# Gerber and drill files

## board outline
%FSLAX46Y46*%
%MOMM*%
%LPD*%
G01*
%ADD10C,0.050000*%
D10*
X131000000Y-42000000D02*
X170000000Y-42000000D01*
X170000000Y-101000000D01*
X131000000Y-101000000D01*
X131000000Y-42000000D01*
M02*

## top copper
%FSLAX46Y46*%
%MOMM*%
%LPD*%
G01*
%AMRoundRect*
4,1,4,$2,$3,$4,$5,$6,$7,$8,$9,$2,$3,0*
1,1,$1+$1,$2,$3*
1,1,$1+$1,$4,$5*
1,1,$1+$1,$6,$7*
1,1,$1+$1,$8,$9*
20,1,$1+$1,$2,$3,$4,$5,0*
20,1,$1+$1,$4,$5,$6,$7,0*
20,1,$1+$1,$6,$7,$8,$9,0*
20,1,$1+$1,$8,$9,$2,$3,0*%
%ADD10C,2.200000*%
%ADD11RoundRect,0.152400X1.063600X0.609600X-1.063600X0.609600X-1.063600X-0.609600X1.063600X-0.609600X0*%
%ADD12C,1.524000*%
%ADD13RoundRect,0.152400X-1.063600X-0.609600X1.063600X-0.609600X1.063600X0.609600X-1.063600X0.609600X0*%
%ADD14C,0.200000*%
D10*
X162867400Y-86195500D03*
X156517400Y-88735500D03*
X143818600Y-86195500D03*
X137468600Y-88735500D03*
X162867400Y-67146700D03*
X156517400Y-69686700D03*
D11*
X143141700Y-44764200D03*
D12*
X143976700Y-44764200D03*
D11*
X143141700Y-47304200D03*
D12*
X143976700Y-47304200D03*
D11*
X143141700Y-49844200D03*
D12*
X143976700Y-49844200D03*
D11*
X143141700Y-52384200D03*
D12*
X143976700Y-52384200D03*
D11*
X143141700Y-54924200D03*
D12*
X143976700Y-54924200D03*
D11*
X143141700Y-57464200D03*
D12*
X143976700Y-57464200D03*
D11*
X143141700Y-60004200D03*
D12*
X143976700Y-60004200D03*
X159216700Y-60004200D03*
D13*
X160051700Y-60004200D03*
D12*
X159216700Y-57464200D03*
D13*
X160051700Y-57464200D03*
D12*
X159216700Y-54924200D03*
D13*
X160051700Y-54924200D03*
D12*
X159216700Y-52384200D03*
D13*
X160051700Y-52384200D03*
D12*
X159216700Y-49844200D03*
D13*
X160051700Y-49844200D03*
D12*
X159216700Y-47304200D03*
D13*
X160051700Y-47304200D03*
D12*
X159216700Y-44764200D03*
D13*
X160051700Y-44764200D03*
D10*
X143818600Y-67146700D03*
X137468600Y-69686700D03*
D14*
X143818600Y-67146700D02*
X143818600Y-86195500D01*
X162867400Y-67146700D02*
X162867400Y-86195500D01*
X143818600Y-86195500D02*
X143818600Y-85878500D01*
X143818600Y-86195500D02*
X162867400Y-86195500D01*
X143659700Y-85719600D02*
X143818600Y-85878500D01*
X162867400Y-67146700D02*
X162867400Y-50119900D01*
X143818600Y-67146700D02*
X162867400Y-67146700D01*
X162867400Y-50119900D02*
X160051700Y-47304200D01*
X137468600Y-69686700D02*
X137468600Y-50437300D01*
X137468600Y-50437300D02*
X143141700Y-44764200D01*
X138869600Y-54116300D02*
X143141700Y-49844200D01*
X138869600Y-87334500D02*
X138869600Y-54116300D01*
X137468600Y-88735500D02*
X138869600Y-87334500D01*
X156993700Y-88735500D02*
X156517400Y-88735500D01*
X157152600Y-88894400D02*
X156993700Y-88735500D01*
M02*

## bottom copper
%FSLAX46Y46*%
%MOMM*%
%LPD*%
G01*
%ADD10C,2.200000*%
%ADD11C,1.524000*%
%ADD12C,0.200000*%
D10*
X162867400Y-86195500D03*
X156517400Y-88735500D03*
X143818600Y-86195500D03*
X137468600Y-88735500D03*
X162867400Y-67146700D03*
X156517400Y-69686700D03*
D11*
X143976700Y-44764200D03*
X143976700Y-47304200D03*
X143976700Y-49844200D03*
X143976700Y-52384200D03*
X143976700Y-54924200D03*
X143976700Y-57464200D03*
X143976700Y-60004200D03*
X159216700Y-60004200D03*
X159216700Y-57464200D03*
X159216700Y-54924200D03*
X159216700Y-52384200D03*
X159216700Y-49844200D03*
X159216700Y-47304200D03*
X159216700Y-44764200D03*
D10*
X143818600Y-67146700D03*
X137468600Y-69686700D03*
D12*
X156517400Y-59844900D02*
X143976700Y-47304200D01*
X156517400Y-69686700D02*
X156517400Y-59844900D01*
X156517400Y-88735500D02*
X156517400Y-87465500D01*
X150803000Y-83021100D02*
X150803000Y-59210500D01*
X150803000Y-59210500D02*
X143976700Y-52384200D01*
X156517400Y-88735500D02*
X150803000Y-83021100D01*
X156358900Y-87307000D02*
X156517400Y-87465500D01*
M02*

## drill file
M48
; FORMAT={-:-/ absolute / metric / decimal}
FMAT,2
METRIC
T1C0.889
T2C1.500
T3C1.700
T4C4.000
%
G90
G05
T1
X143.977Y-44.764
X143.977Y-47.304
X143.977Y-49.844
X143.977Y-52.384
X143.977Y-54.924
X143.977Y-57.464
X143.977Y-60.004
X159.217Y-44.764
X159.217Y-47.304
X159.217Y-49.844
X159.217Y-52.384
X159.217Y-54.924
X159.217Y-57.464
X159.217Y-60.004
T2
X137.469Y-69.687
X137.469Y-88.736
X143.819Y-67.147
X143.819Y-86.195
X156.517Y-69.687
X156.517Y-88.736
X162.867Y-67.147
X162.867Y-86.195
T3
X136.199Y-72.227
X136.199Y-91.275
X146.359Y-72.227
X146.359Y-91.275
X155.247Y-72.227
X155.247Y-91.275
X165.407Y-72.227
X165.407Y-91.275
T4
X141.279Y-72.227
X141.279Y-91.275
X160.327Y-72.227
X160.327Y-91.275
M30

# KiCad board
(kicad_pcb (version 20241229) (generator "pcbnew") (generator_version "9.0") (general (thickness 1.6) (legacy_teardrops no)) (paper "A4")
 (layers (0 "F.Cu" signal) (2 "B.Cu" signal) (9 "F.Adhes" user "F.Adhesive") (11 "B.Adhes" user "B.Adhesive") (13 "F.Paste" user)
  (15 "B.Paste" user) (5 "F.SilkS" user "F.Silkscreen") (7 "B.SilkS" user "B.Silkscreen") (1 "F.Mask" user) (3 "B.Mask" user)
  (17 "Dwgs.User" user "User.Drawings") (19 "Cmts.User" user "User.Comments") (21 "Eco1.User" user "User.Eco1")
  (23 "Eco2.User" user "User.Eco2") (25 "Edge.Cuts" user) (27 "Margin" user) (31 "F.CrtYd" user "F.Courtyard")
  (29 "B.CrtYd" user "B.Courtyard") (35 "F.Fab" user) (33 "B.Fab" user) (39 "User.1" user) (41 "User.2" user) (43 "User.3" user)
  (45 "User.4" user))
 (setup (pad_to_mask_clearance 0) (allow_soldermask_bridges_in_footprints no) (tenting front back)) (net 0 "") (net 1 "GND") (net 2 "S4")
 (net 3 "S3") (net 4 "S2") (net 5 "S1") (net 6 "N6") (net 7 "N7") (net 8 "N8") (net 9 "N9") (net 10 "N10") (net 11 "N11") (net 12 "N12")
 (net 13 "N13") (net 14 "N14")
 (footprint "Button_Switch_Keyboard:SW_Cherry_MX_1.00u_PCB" (layer "F.Cu") (at 162.8674 86.1955)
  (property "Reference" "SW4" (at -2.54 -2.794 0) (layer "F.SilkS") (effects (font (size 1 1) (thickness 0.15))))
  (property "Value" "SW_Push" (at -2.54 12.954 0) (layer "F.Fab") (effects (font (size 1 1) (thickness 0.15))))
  (pad "" np_thru_hole circle (at -7.62 5.08) (size 1.7 1.7) (drill 1.7) (layers "*.Cu" "*.Mask"))
  (pad "" np_thru_hole circle (at -2.54 5.08) (size 4 4) (drill 4) (layers "*.Cu" "*.Mask"))
  (pad "" np_thru_hole circle (at 2.54 5.08) (size 1.7 1.7) (drill 1.7) (layers "*.Cu" "*.Mask"))
  (pad "1" thru_hole circle (at 0 0) (size 2.2 2.2) (drill 1.5) (layers "*.Cu" "*.Mask") (remove_unused_layers no) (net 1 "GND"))
  (pad "2" thru_hole circle (at -6.35 2.54) (size 2.2 2.2) (drill 1.5) (layers "*.Cu" "*.Mask") (remove_unused_layers no) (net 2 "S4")))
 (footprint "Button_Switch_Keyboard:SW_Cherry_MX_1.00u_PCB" (layer "F.Cu") (at 143.8186 86.1955)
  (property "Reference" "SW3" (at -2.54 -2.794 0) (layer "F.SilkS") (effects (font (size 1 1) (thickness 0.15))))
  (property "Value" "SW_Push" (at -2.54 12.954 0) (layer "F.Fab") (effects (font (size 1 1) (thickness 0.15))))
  (pad "" np_thru_hole circle (at -7.62 5.08) (size 1.7 1.7) (drill 1.7) (layers "*.Cu" "*.Mask"))
  (pad "" np_thru_hole circle (at -2.54 5.08) (size 4 4) (drill 4) (layers "*.Cu" "*.Mask"))
  (pad "" np_thru_hole circle (at 2.54 5.08) (size 1.7 1.7) (drill 1.7) (layers "*.Cu" "*.Mask"))
  (pad "1" thru_hole circle (at 0 0) (size 2.2 2.2) (drill 1.5) (layers "*.Cu" "*.Mask") (remove_unused_layers no) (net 1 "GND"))
  (pad "2" thru_hole circle (at -6.35 2.54) (size 2.2 2.2) (drill 1.5) (layers "*.Cu" "*.Mask") (remove_unused_layers no) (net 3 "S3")))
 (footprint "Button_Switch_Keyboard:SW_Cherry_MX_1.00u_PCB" (layer "F.Cu") (at 162.8674 67.1467)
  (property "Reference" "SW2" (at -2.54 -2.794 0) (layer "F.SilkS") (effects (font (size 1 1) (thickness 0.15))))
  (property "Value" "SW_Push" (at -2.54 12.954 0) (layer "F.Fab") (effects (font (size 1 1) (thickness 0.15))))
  (pad "" np_thru_hole circle (at -7.62 5.08) (size 1.7 1.7) (drill 1.7) (layers "*.Cu" "*.Mask"))
  (pad "" np_thru_hole circle (at -2.54 5.08) (size 4 4) (drill 4) (layers "*.Cu" "*.Mask"))
  (pad "" np_thru_hole circle (at 2.54 5.08) (size 1.7 1.7) (drill 1.7) (layers "*.Cu" "*.Mask"))
  (pad "1" thru_hole circle (at 0 0) (size 2.2 2.2) (drill 1.5) (layers "*.Cu" "*.Mask") (remove_unused_layers no) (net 1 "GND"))
  (pad "2" thru_hole circle (at -6.35 2.54) (size 2.2 2.2) (drill 1.5) (layers "*.Cu" "*.Mask") (remove_unused_layers no) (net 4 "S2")))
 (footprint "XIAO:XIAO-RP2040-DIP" (layer "F.Cu") (at 151.5967 52.3842)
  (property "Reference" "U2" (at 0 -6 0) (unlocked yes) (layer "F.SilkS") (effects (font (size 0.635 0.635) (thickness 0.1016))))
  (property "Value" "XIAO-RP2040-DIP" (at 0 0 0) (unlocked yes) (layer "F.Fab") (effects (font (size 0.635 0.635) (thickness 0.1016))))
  (pad "1" smd roundrect (at -8.455 -7.62 180) (size 2.432 1.524) (layers "F.Cu" "F.Mask") (roundrect_rratio 0.1) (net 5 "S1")
   (thermal_bridge_angle 45))
  (pad "1" thru_hole circle (at -7.62 -7.62 180) (size 1.524 1.524) (drill 0.889) (layers "*.Cu" "*.Mask") (remove_unused_layers no)
   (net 5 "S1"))
  (pad "2" smd roundrect (at -8.455 -5.08 180) (size 2.432 1.524) (layers "F.Cu" "F.Mask") (roundrect_rratio 0.1) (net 4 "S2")
   (thermal_bridge_angle 45))
  (pad "2" thru_hole circle (at -7.62 -5.08 180) (size 1.524 1.524) (drill 0.889) (layers "*.Cu" "*.Mask") (remove_unused_layers no)
   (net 4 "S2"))
  (pad "3" smd roundrect (at -8.455 -2.54 180) (size 2.432 1.524) (layers "F.Cu" "F.Mask") (roundrect_rratio 0.1) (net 3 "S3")
   (thermal_bridge_angle 45))
  (pad "3" thru_hole circle (at -7.62 -2.54 180) (size 1.524 1.524) (drill 0.889) (layers "*.Cu" "*.Mask") (remove_unused_layers no)
   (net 3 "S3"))
  (pad "4" smd roundrect (at -8.455 0 180) (size 2.432 1.524) (layers "F.Cu" "F.Mask") (roundrect_rratio 0.1) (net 2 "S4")
   (thermal_bridge_angle 45))
  (pad "4" thru_hole circle (at -7.62 0 180) (size 1.524 1.524) (drill 0.889) (layers "*.Cu" "*.Mask") (remove_unused_layers no)
   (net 2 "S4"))
  (pad "5" smd roundrect (at -8.455 2.54 180) (size 2.432 1.524) (layers "F.Cu" "F.Mask") (roundrect_rratio 0.1) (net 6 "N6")
   (thermal_bridge_angle 45))
  (pad "5" thru_hole circle (at -7.62 2.54 180) (size 1.524 1.524) (drill 0.889) (layers "*.Cu" "*.Mask") (remove_unused_layers no)
   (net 6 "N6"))
  (pad "6" smd roundrect (at -8.455 5.08 180) (size 2.432 1.524) (layers "F.Cu" "F.Mask") (roundrect_rratio 0.1) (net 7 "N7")
   (thermal_bridge_angle 45))
  (pad "6" thru_hole circle (at -7.62 5.08 180) (size 1.524 1.524) (drill 0.889) (layers "*.Cu" "*.Mask") (remove_unused_layers no)
   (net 7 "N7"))
  (pad "7" smd roundrect (at -8.455 7.62 180) (size 2.432 1.524) (layers "F.Cu" "F.Mask") (roundrect_rratio 0.1) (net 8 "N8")
   (thermal_bridge_angle 45))
  (pad "7" thru_hole circle (at -7.62 7.62 180) (size 1.524 1.524) (drill 0.889) (layers "*.Cu" "*.Mask") (remove_unused_layers no)
   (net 8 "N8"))
  (pad "8" thru_hole circle (at 7.62 7.62) (size 1.524 1.524) (drill 0.889) (layers "*.Cu" "*.Mask") (remove_unused_layers no) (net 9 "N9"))
  (pad "8" smd roundrect (at 8.455 7.62) (size 2.432 1.524) (layers "F.Cu" "F.Mask") (roundrect_rratio 0.1) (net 9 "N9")
   (thermal_bridge_angle 45))
  (pad "9" thru_hole circle (at 7.62 5.08) (size 1.524 1.524) (drill 0.889) (layers "*.Cu" "*.Mask") (remove_unused_layers no)
   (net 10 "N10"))
  (pad "9" smd roundrect (at 8.455 5.08) (size 2.432 1.524) (layers "F.Cu" "F.Mask") (roundrect_rratio 0.1) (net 10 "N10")
   (thermal_bridge_angle 45))
  (pad "10" thru_hole circle (at 7.62 2.54) (size 1.524 1.524) (drill 0.889) (layers "*.Cu" "*.Mask") (remove_unused_layers no)
   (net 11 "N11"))
  (pad "10" smd roundrect (at 8.455 2.54) (size 2.432 1.524) (layers "F.Cu" "F.Mask") (roundrect_rratio 0.1) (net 11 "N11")
   (thermal_bridge_angle 45))
  (pad "11" thru_hole circle (at 7.62 0) (size 1.524 1.524) (drill 0.889) (layers "*.Cu" "*.Mask") (remove_unused_layers no) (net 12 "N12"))
  (pad "11" smd roundrect (at 8.455 0) (size 2.432 1.524) (layers "F.Cu" "F.Mask") (roundrect_rratio 0.1) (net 12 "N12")
   (thermal_bridge_angle 45))
  (pad "12" thru_hole circle (at 7.62 -2.54) (size 1.524 1.524) (drill 0.889) (layers "*.Cu" "*.Mask") (remove_unused_layers no)
   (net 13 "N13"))
  (pad "12" smd roundrect (at 8.455 -2.54) (size 2.432 1.524) (layers "F.Cu" "F.Mask") (roundrect_rratio 0.1) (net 13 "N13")
   (thermal_bridge_angle 45))
  (pad "13" thru_hole circle (at 7.62 -5.08) (size 1.524 1.524) (drill 0.889) (layers "*.Cu" "*.Mask") (remove_unused_layers no)
   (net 1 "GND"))
  (pad "13" smd roundrect (at 8.455 -5.08) (size 2.432 1.524) (layers "F.Cu" "F.Mask") (roundrect_rratio 0.1) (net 1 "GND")
   (thermal_bridge_angle 45))
  (pad "14" thru_hole circle (at 7.62 -7.62) (size 1.524 1.524) (drill 0.889) (layers "*.Cu" "*.Mask") (remove_unused_layers no)
   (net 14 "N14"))
  (pad "14" smd roundrect (at 8.455 -7.62) (size 2.432 1.524) (layers "F.Cu" "F.Mask") (roundrect_rratio 0.1) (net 14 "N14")
   (thermal_bridge_angle 45)))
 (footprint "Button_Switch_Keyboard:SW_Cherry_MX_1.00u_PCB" (layer "F.Cu") (at 143.8186 67.1467)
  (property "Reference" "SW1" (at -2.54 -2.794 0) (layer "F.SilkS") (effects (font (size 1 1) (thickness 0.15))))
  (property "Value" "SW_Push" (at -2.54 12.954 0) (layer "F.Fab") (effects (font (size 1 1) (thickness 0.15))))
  (pad "" np_thru_hole circle (at -7.62 5.08) (size 1.7 1.7) (drill 1.7) (layers "*.Cu" "*.Mask"))
  (pad "" np_thru_hole circle (at -2.54 5.08) (size 4 4) (drill 4) (layers "*.Cu" "*.Mask"))
  (pad "" np_thru_hole circle (at 2.54 5.08) (size 1.7 1.7) (drill 1.7) (layers "*.Cu" "*.Mask"))
  (pad "1" thru_hole circle (at 0 0) (size 2.2 2.2) (drill 1.5) (layers "*.Cu" "*.Mask") (remove_unused_layers no) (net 1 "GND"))
  (pad "2" thru_hole circle (at -6.35 2.54) (size 2.2 2.2) (drill 1.5) (layers "*.Cu" "*.Mask") (remove_unused_layers no) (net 5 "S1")))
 (gr_rect (start 131 42) (end 170 101) (stroke (width 0.05) (type default)) (fill no) (layer "Edge.Cuts"))
 (segment (start 143.8186 67.1467) (end 143.8186 86.1955) (width 0.2) (layer "F.Cu") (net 1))
 (segment (start 162.8674 67.1467) (end 162.8674 86.1955) (width 0.2) (layer "F.Cu") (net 1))
 (segment (start 143.8186 86.1955) (end 143.8186 85.8785) (width 0.2) (layer "F.Cu") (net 1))
 (segment (start 143.8186 86.1955) (end 162.8674 86.1955) (width 0.2) (layer "F.Cu") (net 1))
 (segment (start 143.6597 85.7196) (end 143.8186 85.8785) (width 0.2) (layer "F.Cu") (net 1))
 (segment (start 162.8674 67.1467) (end 162.8674 50.1199) (width 0.2) (layer "F.Cu") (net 1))
 (segment (start 143.8186 67.1467) (end 162.8674 67.1467) (width 0.2) (layer "F.Cu") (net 1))
 (segment (start 162.8674 50.1199) (end 160.0517 47.3042) (width 0.2) (layer "F.Cu") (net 1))
 (segment (start 137.4686 69.6867) (end 137.4686 50.4373) (width 0.2) (layer "F.Cu") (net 5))
 (segment (start 137.4686 50.4373) (end 143.1417 44.7642) (width 0.2) (layer "F.Cu") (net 5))
 (segment (start 156.5174 59.8449) (end 143.9767 47.3042) (width 0.2) (layer "B.Cu") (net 4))
 (segment (start 156.5174 69.6867) (end 156.5174 59.8449) (width 0.2) (layer "B.Cu") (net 4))
 (segment (start 138.8696 54.1163) (end 143.1417 49.8442) (width 0.2) (layer "F.Cu") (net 3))
 (segment (start 138.8696 87.3345) (end 138.8696 54.1163) (width 0.2) (layer "F.Cu") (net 3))
 (segment (start 137.4686 88.7355) (end 138.8696 87.3345) (width 0.2) (layer "F.Cu") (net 3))
 (segment (start 156.9937 88.7355) (end 156.5174 88.7355) (width 0.2) (layer "F.Cu") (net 2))
 (segment (start 157.1526 88.8944) (end 156.9937 88.7355) (width 0.2) (layer "F.Cu") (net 2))
 (segment (start 156.5174 88.7355) (end 156.5174 87.4655) (width 0.2) (layer "B.Cu") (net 2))
 (segment (start 150.803 83.0211) (end 150.803 59.2105) (width 0.2) (layer "B.Cu") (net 2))
 (segment (start 150.803 59.2105) (end 143.9767 52.3842) (width 0.2) (layer "B.Cu") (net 2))
 (segment (start 156.5174 88.7355) (end 150.803 83.0211) (width 0.2) (layer "B.Cu") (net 2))
 (segment (start 156.3589 87.307) (end 156.5174 87.4655) (width 0.2) (layer "B.Cu") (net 2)))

